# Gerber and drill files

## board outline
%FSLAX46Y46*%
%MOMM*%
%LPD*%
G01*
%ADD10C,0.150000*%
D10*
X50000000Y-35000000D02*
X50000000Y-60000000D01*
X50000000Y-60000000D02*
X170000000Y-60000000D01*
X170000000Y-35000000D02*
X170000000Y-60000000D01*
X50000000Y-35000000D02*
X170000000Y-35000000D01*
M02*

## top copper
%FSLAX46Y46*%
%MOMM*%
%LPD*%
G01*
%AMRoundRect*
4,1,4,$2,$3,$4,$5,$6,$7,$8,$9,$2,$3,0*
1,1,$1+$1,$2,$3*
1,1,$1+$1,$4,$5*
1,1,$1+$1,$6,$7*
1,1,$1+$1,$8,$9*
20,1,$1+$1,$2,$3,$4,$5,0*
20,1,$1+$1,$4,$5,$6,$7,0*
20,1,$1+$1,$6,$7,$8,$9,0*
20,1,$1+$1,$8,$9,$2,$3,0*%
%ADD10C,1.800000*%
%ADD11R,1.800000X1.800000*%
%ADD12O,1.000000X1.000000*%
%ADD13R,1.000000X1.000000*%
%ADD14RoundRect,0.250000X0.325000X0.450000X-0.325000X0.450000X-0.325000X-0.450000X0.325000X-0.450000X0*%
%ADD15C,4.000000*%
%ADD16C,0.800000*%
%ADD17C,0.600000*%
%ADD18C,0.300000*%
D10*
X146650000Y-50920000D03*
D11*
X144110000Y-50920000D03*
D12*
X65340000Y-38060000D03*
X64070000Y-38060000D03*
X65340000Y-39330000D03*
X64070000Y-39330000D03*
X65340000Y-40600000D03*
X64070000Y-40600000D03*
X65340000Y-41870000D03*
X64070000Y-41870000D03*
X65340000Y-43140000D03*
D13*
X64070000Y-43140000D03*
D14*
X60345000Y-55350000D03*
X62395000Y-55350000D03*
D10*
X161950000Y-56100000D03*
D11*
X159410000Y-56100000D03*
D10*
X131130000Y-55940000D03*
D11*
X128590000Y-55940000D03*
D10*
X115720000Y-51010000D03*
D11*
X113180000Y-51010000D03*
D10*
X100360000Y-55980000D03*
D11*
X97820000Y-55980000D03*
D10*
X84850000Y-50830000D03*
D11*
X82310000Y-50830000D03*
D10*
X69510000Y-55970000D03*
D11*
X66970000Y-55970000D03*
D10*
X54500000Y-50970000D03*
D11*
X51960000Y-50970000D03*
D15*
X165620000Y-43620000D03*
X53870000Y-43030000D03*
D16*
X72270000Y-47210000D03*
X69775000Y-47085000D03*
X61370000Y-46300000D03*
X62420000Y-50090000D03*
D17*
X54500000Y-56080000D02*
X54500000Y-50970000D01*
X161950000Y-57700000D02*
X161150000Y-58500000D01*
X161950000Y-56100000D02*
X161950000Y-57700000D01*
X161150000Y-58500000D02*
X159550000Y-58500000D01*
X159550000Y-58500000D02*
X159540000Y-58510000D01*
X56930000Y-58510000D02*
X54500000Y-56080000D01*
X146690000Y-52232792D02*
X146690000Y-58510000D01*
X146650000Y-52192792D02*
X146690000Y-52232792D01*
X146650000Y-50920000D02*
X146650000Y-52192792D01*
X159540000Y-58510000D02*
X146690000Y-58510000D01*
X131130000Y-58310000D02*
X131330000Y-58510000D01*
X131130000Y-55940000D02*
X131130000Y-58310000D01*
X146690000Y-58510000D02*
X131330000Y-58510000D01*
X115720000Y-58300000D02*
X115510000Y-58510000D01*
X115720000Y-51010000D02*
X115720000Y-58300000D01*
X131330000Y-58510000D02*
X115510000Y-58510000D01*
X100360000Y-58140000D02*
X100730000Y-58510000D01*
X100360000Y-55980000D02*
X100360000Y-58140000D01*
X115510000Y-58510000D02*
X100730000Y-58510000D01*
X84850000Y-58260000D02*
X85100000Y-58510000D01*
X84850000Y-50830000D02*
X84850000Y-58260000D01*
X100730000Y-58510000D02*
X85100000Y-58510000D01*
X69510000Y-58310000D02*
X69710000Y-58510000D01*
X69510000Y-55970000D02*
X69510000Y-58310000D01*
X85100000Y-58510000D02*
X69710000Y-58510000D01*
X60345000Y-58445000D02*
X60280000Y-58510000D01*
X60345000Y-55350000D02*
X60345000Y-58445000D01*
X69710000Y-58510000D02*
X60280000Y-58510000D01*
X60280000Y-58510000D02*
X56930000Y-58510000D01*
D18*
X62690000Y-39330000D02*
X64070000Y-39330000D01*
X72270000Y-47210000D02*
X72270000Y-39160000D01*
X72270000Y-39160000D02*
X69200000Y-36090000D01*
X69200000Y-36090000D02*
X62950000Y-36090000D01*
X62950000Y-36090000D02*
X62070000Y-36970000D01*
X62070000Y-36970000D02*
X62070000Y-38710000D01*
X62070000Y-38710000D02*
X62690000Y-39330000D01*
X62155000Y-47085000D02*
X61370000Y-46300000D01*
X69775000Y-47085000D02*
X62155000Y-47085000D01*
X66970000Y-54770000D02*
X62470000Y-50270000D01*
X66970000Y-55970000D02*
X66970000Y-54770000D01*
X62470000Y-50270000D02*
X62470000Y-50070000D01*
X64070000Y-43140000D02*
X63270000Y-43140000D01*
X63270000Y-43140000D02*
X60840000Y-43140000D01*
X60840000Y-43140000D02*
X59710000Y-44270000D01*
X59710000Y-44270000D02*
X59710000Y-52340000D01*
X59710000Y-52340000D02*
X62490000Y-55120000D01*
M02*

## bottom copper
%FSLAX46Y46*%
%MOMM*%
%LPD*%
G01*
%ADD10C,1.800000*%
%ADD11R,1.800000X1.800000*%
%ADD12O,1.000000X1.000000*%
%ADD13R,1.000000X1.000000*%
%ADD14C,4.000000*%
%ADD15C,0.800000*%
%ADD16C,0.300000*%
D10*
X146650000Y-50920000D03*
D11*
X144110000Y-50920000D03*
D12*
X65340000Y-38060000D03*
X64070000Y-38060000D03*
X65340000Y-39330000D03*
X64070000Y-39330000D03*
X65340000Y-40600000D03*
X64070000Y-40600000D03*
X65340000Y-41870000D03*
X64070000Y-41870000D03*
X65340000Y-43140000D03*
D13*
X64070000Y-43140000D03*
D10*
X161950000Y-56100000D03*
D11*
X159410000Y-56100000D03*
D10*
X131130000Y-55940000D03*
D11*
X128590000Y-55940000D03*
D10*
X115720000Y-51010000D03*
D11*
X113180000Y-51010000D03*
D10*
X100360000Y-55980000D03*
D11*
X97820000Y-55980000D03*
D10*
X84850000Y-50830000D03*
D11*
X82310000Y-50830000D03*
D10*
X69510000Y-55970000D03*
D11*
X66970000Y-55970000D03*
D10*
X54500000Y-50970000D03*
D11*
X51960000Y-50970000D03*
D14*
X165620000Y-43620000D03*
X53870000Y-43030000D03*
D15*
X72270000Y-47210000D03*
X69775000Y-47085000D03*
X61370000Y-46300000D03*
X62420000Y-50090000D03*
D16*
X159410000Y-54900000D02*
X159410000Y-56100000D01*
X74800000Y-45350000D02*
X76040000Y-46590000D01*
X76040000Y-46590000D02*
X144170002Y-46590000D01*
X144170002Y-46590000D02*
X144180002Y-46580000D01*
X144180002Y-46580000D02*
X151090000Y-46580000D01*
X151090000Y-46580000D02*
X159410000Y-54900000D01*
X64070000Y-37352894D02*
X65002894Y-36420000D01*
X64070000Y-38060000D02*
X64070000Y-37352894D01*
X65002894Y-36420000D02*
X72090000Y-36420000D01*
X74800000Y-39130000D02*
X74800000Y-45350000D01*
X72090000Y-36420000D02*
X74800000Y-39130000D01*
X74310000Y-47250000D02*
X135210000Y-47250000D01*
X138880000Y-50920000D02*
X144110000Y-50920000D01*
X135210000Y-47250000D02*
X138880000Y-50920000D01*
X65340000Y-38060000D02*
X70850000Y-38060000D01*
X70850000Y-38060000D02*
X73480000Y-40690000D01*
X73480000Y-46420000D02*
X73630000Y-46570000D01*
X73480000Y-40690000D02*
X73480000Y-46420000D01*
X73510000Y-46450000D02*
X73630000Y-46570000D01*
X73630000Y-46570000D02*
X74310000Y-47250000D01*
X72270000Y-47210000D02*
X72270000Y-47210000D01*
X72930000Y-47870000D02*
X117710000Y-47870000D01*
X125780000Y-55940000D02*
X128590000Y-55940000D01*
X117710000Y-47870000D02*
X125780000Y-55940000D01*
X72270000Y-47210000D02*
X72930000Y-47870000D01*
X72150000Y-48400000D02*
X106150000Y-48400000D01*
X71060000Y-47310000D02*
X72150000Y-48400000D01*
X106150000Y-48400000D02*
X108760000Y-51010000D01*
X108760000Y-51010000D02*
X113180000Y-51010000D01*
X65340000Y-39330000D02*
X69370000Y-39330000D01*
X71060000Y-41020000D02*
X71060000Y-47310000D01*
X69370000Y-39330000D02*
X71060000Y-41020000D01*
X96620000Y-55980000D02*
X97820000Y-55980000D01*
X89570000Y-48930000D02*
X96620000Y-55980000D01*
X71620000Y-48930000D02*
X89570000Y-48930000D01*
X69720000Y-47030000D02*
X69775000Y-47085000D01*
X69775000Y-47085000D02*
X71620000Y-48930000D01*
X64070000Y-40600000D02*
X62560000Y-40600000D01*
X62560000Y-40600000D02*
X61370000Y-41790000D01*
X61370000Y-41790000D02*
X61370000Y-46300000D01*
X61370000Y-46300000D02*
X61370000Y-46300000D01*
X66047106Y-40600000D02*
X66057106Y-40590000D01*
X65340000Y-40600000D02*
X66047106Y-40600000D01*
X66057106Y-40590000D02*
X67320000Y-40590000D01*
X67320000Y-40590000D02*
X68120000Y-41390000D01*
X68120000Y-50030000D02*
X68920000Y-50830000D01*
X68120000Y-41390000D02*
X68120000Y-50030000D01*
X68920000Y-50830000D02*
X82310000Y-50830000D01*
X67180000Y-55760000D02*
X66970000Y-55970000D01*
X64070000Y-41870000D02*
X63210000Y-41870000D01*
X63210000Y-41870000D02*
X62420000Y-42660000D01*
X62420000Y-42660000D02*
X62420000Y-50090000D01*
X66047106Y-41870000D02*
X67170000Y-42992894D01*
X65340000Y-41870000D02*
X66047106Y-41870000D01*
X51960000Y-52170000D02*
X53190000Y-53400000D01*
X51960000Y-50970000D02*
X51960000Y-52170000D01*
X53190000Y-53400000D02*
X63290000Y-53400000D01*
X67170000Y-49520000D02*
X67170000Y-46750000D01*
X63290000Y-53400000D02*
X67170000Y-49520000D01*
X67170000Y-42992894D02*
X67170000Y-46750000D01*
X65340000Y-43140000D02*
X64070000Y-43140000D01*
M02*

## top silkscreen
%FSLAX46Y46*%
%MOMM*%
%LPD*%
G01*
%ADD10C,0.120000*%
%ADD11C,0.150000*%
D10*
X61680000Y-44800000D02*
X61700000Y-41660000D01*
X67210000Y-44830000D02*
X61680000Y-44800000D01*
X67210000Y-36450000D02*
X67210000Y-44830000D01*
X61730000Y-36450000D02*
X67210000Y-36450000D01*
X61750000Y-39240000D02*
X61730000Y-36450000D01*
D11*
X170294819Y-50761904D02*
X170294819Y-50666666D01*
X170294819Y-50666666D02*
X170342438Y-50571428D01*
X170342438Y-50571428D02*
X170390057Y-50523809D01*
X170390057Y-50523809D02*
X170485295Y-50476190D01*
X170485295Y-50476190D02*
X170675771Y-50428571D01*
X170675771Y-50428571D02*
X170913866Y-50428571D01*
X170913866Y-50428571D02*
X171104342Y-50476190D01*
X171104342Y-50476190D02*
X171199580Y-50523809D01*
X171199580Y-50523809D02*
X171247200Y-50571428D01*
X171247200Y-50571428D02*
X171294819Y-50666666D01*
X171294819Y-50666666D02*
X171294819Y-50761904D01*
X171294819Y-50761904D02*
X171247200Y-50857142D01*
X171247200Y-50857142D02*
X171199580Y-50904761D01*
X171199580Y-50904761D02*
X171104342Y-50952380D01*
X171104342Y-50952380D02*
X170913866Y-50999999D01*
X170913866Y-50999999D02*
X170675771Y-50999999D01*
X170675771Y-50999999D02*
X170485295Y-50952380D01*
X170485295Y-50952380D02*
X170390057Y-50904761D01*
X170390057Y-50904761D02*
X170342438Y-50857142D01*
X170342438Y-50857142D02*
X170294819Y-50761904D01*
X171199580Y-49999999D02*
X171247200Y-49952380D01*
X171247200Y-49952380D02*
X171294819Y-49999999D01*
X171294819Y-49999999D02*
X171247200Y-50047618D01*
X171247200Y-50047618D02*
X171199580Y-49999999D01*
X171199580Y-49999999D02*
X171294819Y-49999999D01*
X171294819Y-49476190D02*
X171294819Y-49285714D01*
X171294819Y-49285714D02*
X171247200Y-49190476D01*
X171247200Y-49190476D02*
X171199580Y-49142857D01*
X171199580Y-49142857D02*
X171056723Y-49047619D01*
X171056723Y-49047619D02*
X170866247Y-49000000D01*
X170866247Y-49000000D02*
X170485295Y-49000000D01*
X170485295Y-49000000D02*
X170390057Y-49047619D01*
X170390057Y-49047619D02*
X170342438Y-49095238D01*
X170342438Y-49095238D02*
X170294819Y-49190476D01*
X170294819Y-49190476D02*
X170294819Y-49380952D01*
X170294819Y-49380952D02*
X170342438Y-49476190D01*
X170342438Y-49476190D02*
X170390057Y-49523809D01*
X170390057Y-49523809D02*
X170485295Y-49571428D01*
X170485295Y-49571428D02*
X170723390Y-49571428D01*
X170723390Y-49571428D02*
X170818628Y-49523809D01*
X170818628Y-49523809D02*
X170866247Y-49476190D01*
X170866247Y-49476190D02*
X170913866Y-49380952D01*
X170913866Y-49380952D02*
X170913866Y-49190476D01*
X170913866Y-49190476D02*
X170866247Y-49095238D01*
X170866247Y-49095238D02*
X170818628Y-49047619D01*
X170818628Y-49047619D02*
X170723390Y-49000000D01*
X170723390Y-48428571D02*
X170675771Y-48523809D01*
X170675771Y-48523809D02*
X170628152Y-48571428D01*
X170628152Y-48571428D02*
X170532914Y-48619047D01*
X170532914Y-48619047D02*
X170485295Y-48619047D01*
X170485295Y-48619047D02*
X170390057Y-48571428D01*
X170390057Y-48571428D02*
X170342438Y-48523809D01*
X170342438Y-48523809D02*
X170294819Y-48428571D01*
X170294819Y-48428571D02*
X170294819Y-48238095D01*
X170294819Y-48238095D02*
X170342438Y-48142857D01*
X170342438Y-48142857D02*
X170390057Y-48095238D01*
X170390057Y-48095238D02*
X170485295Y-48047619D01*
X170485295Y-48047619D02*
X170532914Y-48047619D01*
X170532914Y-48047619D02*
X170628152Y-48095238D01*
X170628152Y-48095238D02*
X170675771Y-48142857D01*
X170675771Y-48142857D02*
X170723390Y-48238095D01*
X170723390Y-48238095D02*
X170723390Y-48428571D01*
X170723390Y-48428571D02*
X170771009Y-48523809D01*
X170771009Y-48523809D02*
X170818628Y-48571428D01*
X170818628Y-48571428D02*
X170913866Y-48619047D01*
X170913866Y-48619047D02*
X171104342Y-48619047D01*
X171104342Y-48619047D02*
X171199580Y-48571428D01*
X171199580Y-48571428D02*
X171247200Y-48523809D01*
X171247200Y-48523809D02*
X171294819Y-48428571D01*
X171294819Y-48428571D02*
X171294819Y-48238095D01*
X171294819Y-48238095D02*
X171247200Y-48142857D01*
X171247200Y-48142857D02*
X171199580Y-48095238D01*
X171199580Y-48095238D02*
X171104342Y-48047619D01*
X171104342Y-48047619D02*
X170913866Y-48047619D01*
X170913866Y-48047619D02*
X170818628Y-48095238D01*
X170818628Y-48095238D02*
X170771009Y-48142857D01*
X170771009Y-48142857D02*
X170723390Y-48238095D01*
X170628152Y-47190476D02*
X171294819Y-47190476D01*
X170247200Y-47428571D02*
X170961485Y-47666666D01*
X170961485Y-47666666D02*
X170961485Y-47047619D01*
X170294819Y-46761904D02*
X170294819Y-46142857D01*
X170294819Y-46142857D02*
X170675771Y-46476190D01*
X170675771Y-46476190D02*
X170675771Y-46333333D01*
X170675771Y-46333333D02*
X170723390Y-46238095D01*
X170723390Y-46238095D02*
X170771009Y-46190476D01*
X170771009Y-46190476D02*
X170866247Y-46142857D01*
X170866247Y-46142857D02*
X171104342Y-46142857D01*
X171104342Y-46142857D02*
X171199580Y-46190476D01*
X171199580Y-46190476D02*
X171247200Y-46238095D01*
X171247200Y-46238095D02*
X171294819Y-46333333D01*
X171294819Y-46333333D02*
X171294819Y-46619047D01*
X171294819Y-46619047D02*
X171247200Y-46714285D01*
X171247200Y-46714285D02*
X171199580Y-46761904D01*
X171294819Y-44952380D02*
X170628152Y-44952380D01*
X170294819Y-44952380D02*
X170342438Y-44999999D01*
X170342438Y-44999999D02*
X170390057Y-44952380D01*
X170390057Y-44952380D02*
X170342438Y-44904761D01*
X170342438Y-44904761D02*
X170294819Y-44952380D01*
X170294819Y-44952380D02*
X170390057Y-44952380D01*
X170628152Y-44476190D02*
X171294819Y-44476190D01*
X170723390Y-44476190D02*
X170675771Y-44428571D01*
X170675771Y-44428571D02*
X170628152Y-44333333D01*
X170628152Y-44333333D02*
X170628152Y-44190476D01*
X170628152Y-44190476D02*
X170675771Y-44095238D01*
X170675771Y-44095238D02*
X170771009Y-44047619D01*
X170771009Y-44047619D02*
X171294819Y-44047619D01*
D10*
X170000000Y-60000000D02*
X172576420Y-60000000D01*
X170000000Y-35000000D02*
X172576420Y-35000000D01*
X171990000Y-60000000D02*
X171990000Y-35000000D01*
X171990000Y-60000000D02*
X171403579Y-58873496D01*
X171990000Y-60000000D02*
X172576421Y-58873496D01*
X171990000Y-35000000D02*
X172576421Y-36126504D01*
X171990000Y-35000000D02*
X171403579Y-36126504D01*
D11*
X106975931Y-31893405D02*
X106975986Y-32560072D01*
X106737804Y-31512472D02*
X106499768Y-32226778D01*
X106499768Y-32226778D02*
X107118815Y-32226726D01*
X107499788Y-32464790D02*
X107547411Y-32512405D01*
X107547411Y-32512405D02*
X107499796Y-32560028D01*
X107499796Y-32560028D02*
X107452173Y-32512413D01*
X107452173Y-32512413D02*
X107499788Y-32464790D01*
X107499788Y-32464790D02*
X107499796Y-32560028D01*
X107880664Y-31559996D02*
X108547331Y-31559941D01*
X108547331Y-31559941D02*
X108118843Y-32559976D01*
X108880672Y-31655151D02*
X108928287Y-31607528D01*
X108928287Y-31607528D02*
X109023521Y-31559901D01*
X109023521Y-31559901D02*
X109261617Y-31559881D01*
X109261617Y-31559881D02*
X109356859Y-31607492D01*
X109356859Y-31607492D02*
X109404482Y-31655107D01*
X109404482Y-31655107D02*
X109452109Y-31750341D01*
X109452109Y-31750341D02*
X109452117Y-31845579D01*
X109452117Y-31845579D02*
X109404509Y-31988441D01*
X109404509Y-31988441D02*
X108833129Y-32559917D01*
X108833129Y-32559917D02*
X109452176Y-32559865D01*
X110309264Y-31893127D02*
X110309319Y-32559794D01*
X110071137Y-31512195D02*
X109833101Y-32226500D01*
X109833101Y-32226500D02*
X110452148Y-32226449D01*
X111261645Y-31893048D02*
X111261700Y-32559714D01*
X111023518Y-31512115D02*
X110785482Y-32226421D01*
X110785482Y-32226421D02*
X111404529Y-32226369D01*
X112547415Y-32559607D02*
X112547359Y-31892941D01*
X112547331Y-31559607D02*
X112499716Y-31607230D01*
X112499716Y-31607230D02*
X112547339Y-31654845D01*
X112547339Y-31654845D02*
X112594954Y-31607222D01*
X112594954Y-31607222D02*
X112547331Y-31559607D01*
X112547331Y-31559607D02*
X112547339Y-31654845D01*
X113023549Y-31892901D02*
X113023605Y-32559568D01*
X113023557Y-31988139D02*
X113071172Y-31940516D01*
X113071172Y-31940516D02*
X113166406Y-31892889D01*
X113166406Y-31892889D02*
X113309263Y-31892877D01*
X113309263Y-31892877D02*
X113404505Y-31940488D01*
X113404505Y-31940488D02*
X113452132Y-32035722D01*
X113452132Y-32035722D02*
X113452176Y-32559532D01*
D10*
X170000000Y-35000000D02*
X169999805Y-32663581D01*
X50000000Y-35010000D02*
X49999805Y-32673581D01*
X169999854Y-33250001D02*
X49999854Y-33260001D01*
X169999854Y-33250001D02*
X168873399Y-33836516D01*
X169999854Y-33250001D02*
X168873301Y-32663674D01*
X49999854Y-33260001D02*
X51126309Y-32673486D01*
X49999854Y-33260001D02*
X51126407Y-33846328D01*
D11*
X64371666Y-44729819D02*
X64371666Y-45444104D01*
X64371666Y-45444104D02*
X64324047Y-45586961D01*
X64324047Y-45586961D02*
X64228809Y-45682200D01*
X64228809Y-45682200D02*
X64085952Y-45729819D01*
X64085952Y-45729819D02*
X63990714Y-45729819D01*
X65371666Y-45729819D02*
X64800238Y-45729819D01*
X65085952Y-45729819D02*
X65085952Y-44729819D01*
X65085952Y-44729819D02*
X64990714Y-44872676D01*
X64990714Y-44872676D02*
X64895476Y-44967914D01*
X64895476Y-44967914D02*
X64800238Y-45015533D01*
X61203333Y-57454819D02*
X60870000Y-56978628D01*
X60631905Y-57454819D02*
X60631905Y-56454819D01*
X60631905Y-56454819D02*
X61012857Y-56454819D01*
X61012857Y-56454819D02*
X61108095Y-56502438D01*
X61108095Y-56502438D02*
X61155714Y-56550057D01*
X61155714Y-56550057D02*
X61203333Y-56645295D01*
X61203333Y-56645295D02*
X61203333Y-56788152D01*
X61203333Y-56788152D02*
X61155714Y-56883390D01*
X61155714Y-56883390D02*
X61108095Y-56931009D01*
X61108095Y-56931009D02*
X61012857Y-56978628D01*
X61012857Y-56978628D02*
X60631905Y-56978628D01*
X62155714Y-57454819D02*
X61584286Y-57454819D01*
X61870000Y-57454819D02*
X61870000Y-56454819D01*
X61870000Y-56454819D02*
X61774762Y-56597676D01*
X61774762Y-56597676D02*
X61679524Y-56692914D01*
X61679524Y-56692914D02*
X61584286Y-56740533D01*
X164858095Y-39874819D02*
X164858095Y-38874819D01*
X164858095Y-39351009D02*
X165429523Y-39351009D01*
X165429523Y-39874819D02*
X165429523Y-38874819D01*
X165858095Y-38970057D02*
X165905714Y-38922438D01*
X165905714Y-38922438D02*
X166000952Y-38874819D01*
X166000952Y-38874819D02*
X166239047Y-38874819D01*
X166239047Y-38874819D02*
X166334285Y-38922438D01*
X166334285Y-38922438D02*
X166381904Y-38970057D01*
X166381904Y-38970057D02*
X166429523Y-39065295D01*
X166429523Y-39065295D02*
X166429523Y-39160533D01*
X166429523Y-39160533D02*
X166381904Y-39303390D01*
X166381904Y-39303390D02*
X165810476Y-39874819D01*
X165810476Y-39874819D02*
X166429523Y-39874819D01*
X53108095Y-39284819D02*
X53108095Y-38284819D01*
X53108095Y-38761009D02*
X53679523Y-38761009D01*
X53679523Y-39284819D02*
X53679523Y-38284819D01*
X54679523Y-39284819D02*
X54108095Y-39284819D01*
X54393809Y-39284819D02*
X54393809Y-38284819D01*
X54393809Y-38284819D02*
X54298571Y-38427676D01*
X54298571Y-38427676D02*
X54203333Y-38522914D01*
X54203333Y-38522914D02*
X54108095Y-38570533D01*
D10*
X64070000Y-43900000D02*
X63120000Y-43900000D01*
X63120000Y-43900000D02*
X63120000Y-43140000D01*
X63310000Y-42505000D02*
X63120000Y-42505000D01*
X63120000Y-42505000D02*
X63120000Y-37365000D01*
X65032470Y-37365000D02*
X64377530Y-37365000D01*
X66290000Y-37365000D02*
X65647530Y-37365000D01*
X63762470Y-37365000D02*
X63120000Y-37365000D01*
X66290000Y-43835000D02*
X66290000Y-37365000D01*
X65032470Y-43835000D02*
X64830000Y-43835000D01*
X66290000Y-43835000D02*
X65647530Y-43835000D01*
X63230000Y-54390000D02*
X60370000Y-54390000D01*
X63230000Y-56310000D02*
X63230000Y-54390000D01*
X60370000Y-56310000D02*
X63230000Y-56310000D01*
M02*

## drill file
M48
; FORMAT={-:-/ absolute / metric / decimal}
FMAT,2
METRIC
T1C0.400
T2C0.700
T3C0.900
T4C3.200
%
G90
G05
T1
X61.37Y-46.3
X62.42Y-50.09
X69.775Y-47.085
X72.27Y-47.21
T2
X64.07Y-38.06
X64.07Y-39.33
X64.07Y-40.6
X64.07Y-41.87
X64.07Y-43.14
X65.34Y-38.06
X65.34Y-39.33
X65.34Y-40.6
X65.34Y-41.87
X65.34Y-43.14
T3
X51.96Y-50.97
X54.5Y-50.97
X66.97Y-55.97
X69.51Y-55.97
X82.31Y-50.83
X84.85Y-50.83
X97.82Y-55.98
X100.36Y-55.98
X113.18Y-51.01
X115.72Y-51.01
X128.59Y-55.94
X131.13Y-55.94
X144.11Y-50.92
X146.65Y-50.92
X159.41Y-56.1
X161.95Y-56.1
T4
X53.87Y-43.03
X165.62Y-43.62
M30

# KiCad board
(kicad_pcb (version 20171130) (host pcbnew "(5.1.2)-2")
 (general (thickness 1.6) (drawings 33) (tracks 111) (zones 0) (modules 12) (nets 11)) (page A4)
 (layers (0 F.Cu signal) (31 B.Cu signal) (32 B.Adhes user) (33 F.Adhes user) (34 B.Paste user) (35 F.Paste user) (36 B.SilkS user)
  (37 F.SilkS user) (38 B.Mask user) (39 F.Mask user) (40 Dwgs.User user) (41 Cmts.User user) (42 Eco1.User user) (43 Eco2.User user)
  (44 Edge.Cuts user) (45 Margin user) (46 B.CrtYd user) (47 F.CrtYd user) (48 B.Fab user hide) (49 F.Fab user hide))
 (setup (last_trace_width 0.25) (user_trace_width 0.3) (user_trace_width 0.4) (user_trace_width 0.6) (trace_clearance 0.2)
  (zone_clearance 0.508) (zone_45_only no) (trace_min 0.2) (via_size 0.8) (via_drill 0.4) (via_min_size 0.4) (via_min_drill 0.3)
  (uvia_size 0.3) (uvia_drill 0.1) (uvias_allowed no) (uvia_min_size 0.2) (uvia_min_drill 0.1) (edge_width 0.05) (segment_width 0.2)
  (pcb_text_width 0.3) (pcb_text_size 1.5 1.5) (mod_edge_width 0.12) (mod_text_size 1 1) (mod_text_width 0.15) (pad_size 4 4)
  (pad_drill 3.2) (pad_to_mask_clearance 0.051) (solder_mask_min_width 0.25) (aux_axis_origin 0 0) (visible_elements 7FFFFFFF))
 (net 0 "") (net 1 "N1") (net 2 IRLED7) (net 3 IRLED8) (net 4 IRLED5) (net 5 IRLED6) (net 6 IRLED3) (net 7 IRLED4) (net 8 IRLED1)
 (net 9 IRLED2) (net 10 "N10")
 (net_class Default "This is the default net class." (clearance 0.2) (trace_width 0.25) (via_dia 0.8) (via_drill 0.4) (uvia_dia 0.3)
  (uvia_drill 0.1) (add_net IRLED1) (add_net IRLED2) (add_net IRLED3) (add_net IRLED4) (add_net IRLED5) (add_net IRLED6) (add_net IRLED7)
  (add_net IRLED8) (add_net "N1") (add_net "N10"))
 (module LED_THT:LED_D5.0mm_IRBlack (layer B.Cu) (at 144.11 50.92)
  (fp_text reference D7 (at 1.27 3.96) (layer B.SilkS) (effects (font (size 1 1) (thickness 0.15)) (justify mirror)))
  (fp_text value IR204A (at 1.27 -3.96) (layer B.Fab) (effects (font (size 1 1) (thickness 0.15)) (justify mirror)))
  (pad 2 thru_hole circle (at 2.54 0) (size 1.8 1.8) (drill 0.9) (layers *.Cu *.Mask) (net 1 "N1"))
  (pad 1 thru_hole rect (at 0 0) (size 1.8 1.8) (drill 0.9) (layers *.Cu *.Mask) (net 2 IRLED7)))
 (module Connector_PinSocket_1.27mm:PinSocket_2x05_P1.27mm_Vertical (layer F.Cu) (at 64.07 43.14 180)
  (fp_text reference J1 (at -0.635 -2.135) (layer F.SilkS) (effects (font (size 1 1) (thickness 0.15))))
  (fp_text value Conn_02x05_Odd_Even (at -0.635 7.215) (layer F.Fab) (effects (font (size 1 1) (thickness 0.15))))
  (fp_line (start 0 -0.76) (end 0.95 -0.76) (layer F.SilkS) (width 0.12))
  (fp_line (start 0.95 -0.76) (end 0.95 0) (layer F.SilkS) (width 0.12))
  (fp_line (start 0.76 0.635) (end 0.95 0.635) (layer F.SilkS) (width 0.12))
  (fp_line (start 0.95 0.635) (end 0.95 5.775) (layer F.SilkS) (width 0.12))
  (fp_line (start -0.96247 5.775) (end -0.30753 5.775) (layer F.SilkS) (width 0.12))
  (fp_line (start -2.22 5.775) (end -1.57753 5.775) (layer F.SilkS) (width 0.12))
  (fp_line (start 0.30753 5.775) (end 0.95 5.775) (layer F.SilkS) (width 0.12))
  (fp_line (start -2.22 -0.695) (end -2.22 5.775) (layer F.SilkS) (width 0.12))
  (fp_line (start -0.96247 -0.695) (end -0.76 -0.695) (layer F.SilkS) (width 0.12))
  (fp_line (start -2.22 -0.695) (end -1.57753 -0.695) (layer F.SilkS) (width 0.12))
  (pad 10 thru_hole oval (at -1.27 5.08 180) (size 1 1) (drill 0.7) (layers *.Cu *.Mask) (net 2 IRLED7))
  (pad 9 thru_hole oval (at 0 5.08 180) (size 1 1) (drill 0.7) (layers *.Cu *.Mask) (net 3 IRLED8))
  (pad 8 thru_hole oval (at -1.27 3.81 180) (size 1 1) (drill 0.7) (layers *.Cu *.Mask) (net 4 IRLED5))
  (pad 7 thru_hole oval (at 0 3.81 180) (size 1 1) (drill 0.7) (layers *.Cu *.Mask) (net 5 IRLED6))
  (pad 6 thru_hole oval (at -1.27 2.54 180) (size 1 1) (drill 0.7) (layers *.Cu *.Mask) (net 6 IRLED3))
  (pad 5 thru_hole oval (at 0 2.54 180) (size 1 1) (drill 0.7) (layers *.Cu *.Mask) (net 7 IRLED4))
  (pad 4 thru_hole oval (at -1.27 1.27 180) (size 1 1) (drill 0.7) (layers *.Cu *.Mask) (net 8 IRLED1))
  (pad 3 thru_hole oval (at 0 1.27 180) (size 1 1) (drill 0.7) (layers *.Cu *.Mask) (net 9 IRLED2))
  (pad 2 thru_hole oval (at -1.27 0 180) (size 1 1) (drill 0.7) (layers *.Cu *.Mask) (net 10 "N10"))
  (pad 1 thru_hole rect (at 0 0 180) (size 1 1) (drill 0.7) (layers *.Cu *.Mask) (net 10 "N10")))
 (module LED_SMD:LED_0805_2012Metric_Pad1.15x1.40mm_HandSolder (layer F.Cu) (at 61.37 55.35 180)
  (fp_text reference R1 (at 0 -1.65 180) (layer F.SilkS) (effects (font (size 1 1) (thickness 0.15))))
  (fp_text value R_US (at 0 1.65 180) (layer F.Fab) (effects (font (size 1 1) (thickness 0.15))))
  (fp_line (start -1.86 0.96) (end 1 0.96) (layer F.SilkS) (width 0.12))
  (fp_line (start -1.86 -0.96) (end -1.86 0.96) (layer F.SilkS) (width 0.12))
  (fp_line (start 1 -0.96) (end -1.86 -0.96) (layer F.SilkS) (width 0.12))
  (pad 2 smd roundrect (at 1.025 0 180) (size 1.15 1.4) (layers F.Cu F.Paste F.Mask) (roundrect_rratio 0.217391) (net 1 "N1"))
  (pad 1 smd roundrect (at -1.025 0 180) (size 1.15 1.4) (layers F.Cu F.Paste F.Mask) (roundrect_rratio 0.217391) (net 10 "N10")))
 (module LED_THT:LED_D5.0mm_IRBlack (layer B.Cu) (at 159.41 56.1)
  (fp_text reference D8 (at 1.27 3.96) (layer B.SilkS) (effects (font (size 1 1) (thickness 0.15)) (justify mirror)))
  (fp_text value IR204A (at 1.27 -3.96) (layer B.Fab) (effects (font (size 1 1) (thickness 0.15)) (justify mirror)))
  (pad 2 thru_hole circle (at 2.54 0) (size 1.8 1.8) (drill 0.9) (layers *.Cu *.Mask) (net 1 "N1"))
  (pad 1 thru_hole rect (at 0 0) (size 1.8 1.8) (drill 0.9) (layers *.Cu *.Mask) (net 3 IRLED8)))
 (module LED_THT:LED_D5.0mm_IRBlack (layer B.Cu) (at 128.59 55.94)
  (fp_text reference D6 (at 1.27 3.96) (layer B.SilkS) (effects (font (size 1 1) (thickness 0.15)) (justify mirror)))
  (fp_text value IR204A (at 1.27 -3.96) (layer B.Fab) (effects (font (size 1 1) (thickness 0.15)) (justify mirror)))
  (pad 2 thru_hole circle (at 2.54 0) (size 1.8 1.8) (drill 0.9) (layers *.Cu *.Mask) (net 1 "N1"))
  (pad 1 thru_hole rect (at 0 0) (size 1.8 1.8) (drill 0.9) (layers *.Cu *.Mask) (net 5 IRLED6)))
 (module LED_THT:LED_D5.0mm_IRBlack (layer B.Cu) (at 113.18 51.01)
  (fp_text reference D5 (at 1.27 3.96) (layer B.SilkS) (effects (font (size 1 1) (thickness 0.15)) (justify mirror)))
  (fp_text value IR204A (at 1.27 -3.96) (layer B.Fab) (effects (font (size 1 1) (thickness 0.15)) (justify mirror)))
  (pad 2 thru_hole circle (at 2.54 0) (size 1.8 1.8) (drill 0.9) (layers *.Cu *.Mask) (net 1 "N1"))
  (pad 1 thru_hole rect (at 0 0) (size 1.8 1.8) (drill 0.9) (layers *.Cu *.Mask) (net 4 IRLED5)))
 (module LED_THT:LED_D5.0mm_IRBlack (layer B.Cu) (at 97.82 55.98)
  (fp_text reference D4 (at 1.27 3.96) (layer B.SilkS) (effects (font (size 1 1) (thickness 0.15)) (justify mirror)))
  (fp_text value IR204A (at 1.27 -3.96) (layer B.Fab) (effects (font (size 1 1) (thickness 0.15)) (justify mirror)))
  (pad 2 thru_hole circle (at 2.54 0) (size 1.8 1.8) (drill 0.9) (layers *.Cu *.Mask) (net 1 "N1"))
  (pad 1 thru_hole rect (at 0 0) (size 1.8 1.8) (drill 0.9) (layers *.Cu *.Mask) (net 7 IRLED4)))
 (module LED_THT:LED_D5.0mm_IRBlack (layer B.Cu) (at 82.31 50.83)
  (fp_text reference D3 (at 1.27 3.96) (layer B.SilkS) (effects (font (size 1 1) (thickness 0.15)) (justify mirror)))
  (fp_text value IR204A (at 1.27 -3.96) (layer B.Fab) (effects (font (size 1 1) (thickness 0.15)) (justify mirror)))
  (pad 2 thru_hole circle (at 2.54 0) (size 1.8 1.8) (drill 0.9) (layers *.Cu *.Mask) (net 1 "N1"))
  (pad 1 thru_hole rect (at 0 0) (size 1.8 1.8) (drill 0.9) (layers *.Cu *.Mask) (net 6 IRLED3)))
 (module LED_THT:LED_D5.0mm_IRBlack (layer B.Cu) (at 66.97 55.97)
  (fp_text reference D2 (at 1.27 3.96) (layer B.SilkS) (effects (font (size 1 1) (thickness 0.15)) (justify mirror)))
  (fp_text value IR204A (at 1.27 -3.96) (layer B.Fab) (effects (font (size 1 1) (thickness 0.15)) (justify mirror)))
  (pad 2 thru_hole circle (at 2.54 0) (size 1.8 1.8) (drill 0.9) (layers *.Cu *.Mask) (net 1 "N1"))
  (pad 1 thru_hole rect (at 0 0) (size 1.8 1.8) (drill 0.9) (layers *.Cu *.Mask) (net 9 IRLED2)))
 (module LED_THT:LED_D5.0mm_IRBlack (layer B.Cu) (at 51.96 50.97)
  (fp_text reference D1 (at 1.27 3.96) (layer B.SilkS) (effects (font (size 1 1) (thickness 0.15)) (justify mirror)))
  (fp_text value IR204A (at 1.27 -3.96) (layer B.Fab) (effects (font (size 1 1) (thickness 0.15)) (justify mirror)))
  (pad 2 thru_hole circle (at 2.54 0) (size 1.8 1.8) (drill 0.9) (layers *.Cu *.Mask) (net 1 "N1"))
  (pad 1 thru_hole rect (at 0 0) (size 1.8 1.8) (drill 0.9) (layers *.Cu *.Mask) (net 8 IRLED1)))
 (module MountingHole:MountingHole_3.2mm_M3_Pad (layer F.Cu) (at 165.62 43.62)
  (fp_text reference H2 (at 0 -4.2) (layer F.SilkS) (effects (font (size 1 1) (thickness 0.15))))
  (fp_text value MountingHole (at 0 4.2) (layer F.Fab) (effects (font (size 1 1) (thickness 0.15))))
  (pad 1 thru_hole circle (at 0 0) (size 4 4) (drill 3.2) (layers *.Cu *.Mask)))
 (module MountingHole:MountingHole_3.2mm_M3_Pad (layer F.Cu) (at 53.87 43.03)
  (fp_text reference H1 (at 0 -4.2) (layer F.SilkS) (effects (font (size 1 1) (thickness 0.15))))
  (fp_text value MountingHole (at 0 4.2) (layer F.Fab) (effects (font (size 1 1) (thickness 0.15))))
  (pad 1 thru_hole circle (at 0 0) (size 4 4) (drill 3.2) (layers *.Cu *.Mask)))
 (gr_line (start 61.68 44.8) (end 61.7 41.66) (layer F.SilkS) (width 0.12))
 (gr_line (start 67.21 44.83) (end 61.68 44.8) (layer F.SilkS) (width 0.12))
 (gr_line (start 67.21 36.45) (end 67.21 44.83) (layer F.SilkS) (width 0.12))
 (gr_line (start 61.73 36.45) (end 67.21 36.45) (layer F.SilkS) (width 0.12))
 (gr_line (start 61.75 39.24) (end 61.73 36.45) (layer F.SilkS) (width 0.12))
 (gr_line (start 50 35) (end 50 60) (layer Edge.Cuts) (width 0.15))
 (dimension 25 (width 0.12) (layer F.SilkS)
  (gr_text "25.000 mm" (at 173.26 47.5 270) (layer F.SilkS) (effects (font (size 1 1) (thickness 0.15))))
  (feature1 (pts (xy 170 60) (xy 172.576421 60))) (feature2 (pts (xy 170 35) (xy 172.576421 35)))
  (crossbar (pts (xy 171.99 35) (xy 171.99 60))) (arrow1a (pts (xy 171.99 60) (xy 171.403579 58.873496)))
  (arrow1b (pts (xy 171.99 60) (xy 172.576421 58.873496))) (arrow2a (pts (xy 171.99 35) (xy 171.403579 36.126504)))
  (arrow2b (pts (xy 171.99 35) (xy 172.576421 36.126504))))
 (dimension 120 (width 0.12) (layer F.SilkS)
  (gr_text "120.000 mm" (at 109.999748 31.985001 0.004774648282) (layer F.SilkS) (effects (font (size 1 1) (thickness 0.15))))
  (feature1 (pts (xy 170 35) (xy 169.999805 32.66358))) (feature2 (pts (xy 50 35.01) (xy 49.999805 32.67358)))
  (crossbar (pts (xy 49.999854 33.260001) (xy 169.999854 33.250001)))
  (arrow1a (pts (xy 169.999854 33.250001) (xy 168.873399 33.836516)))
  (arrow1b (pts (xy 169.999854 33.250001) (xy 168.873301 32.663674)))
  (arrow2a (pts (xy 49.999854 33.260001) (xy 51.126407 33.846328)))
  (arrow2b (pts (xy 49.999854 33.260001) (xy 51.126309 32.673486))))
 (gr_line (start 50 60) (end 170 60) (layer Edge.Cuts) (width 0.15))
 (gr_line (start 170 35) (end 170 60) (layer Edge.Cuts) (width 0.15))
 (gr_line (start 50 35) (end 170 35) (layer Edge.Cuts) (width 0.15))
 (segment (start 54.5 56.08) (end 54.5 50.97) (width 0.6) (layer F.Cu) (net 1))
 (segment (start 161.95 57.7) (end 161.15 58.5) (width 0.6) (layer F.Cu) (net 1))
 (segment (start 161.95 56.1) (end 161.95 57.7) (width 0.6) (layer F.Cu) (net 1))
 (segment (start 161.15 58.5) (end 159.55 58.5) (width 0.6) (layer F.Cu) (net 1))
 (segment (start 159.55 58.5) (end 159.54 58.51) (width 0.6) (layer F.Cu) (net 1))
 (segment (start 56.93 58.51) (end 54.5 56.08) (width 0.6) (layer F.Cu) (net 1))
 (segment (start 146.69 52.232792) (end 146.69 58.51) (width 0.6) (layer F.Cu) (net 1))
 (segment (start 146.65 52.192792) (end 146.69 52.232792) (width 0.6) (layer F.Cu) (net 1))
 (segment (start 146.65 50.92) (end 146.65 52.192792) (width 0.6) (layer F.Cu) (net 1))
 (segment (start 159.54 58.51) (end 146.69 58.51) (width 0.6) (layer F.Cu) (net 1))
 (segment (start 131.13 58.31) (end 131.33 58.51) (width 0.6) (layer F.Cu) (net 1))
 (segment (start 131.13 55.94) (end 131.13 58.31) (width 0.6) (layer F.Cu) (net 1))
 (segment (start 146.69 58.51) (end 131.33 58.51) (width 0.6) (layer F.Cu) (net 1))
 (segment (start 115.72 58.3) (end 115.51 58.51) (width 0.6) (layer F.Cu) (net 1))
 (segment (start 115.72 51.01) (end 115.72 58.3) (width 0.6) (layer F.Cu) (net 1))
 (segment (start 131.33 58.51) (end 115.51 58.51) (width 0.6) (layer F.Cu) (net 1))
 (segment (start 100.36 58.14) (end 100.73 58.51) (width 0.6) (layer F.Cu) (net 1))
 (segment (start 100.36 55.98) (end 100.36 58.14) (width 0.6) (layer F.Cu) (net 1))
 (segment (start 115.51 58.51) (end 100.73 58.51) (width 0.6) (layer F.Cu) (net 1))
 (segment (start 84.85 58.26) (end 85.1 58.51) (width 0.6) (layer F.Cu) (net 1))
 (segment (start 84.85 50.83) (end 84.85 58.26) (width 0.6) (layer F.Cu) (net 1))
 (segment (start 100.73 58.51) (end 85.1 58.51) (width 0.6) (layer F.Cu) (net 1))
 (segment (start 69.51 58.31) (end 69.71 58.51) (width 0.6) (layer F.Cu) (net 1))
 (segment (start 69.51 55.97) (end 69.51 58.31) (width 0.6) (layer F.Cu) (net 1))
 (segment (start 85.1 58.51) (end 69.71 58.51) (width 0.6) (layer F.Cu) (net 1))
 (segment (start 60.345 58.445) (end 60.28 58.51) (width 0.6) (layer F.Cu) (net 1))
 (segment (start 60.345 55.35) (end 60.345 58.445) (width 0.6) (layer F.Cu) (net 1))
 (segment (start 69.71 58.51) (end 60.28 58.51) (width 0.6) (layer F.Cu) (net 1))
 (segment (start 60.28 58.51) (end 56.93 58.51) (width 0.6) (layer F.Cu) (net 1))
 (segment (start 159.41 54.9) (end 159.41 56.1) (width 0.3) (layer B.Cu) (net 3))
 (segment (start 74.8 45.35) (end 76.04 46.59) (width 0.3) (layer B.Cu) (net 3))
 (segment (start 76.04 46.59) (end 144.170002 46.59) (width 0.3) (layer B.Cu) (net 3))
 (segment (start 144.170002 46.59) (end 144.180002 46.58) (width 0.3) (layer B.Cu) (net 3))
 (segment (start 144.180002 46.58) (end 151.09 46.58) (width 0.3) (layer B.Cu) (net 3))
 (segment (start 151.09 46.58) (end 159.41 54.9) (width 0.3) (layer B.Cu) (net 3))
 (segment (start 64.07 37.352894) (end 65.002894 36.42) (width 0.3) (layer B.Cu) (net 3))
 (segment (start 64.07 38.06) (end 64.07 37.352894) (width 0.3) (layer B.Cu) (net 3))
 (segment (start 65.002894 36.42) (end 72.09 36.42) (width 0.3) (layer B.Cu) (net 3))
 (segment (start 74.8 39.13) (end 74.8 45.35) (width 0.3) (layer B.Cu) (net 3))
 (segment (start 72.09 36.42) (end 74.8 39.13) (width 0.3) (layer B.Cu) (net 3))
 (segment (start 74.31 47.25) (end 135.21 47.25) (width 0.3) (layer B.Cu) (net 2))
 (segment (start 138.88 50.92) (end 144.11 50.92) (width 0.3) (layer B.Cu) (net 2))
 (segment (start 135.21 47.25) (end 138.88 50.92) (width 0.3) (layer B.Cu) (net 2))
 (segment (start 65.34 38.06) (end 70.85 38.06) (width 0.3) (layer B.Cu) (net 2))
 (segment (start 70.85 38.06) (end 73.48 40.69) (width 0.3) (layer B.Cu) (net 2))
 (segment (start 73.48 46.42) (end 73.63 46.57) (width 0.3) (layer B.Cu) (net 2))
 (segment (start 73.48 40.69) (end 73.48 46.42) (width 0.3) (layer B.Cu) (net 2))
 (segment (start 73.51 46.45) (end 73.63 46.57) (width 0.3) (layer B.Cu) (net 2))
 (segment (start 73.63 46.57) (end 74.31 47.25) (width 0.3) (layer B.Cu) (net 2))
 (segment (start 72.27 47.21) (end 72.27 47.21) (width 0.3) (layer B.Cu) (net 5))
 (segment (start 72.93 47.87) (end 117.71 47.87) (width 0.3) (layer B.Cu) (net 5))
 (segment (start 125.78 55.94) (end 128.59 55.94) (width 0.3) (layer B.Cu) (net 5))
 (segment (start 117.71 47.87) (end 125.78 55.94) (width 0.3) (layer B.Cu) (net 5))
 (segment (start 72.27 47.21) (end 72.93 47.87) (width 0.3) (layer B.Cu) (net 5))
 (via (at 72.27 47.21) (size 0.8) (drill 0.4) (layers F.Cu B.Cu) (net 5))
 (segment (start 62.69 39.33) (end 64.07 39.33) (width 0.3) (layer F.Cu) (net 5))
 (segment (start 72.27 47.21) (end 72.27 39.16) (width 0.3) (layer F.Cu) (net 5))
 (segment (start 72.27 39.16) (end 69.2 36.09) (width 0.3) (layer F.Cu) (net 5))
 (segment (start 69.2 36.09) (end 62.95 36.09) (width 0.3) (layer F.Cu) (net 5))
 (segment (start 62.95 36.09) (end 62.07 36.97) (width 0.3) (layer F.Cu) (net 5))
 (segment (start 62.07 36.97) (end 62.07 38.71) (width 0.3) (layer F.Cu) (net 5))
 (segment (start 62.07 38.71) (end 62.69 39.33) (width 0.3) (layer F.Cu) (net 5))
 (segment (start 72.15 48.4) (end 106.15 48.4) (width 0.3) (layer B.Cu) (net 4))
 (segment (start 71.06 47.31) (end 72.15 48.4) (width 0.3) (layer B.Cu) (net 4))
 (segment (start 106.15 48.4) (end 108.76 51.01) (width 0.3) (layer B.Cu) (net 4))
 (segment (start 108.76 51.01) (end 113.18 51.01) (width 0.3) (layer B.Cu) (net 4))
 (segment (start 65.34 39.33) (end 69.37 39.33) (width 0.3) (layer B.Cu) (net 4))
 (segment (start 71.06 41.02) (end 71.06 47.31) (width 0.3) (layer B.Cu) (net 4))
 (segment (start 69.37 39.33) (end 71.06 41.02) (width 0.3) (layer B.Cu) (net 4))
 (segment (start 96.62 55.98) (end 97.82 55.98) (width 0.3) (layer B.Cu) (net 7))
 (segment (start 89.57 48.93) (end 96.62 55.98) (width 0.3) (layer B.Cu) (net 7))
 (segment (start 71.62 48.93) (end 89.57 48.93) (width 0.3) (layer B.Cu) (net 7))
 (segment (start 69.72 47.03) (end 69.775 47.085) (width 0.3) (layer B.Cu) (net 7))
 (segment (start 69.775 47.085) (end 71.62 48.93) (width 0.3) (layer B.Cu) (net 7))
 (via (at 69.775 47.085) (size 0.8) (drill 0.4) (layers F.Cu B.Cu) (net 7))
 (segment (start 64.07 40.6) (end 62.56 40.6) (width 0.3) (layer B.Cu) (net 7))
 (segment (start 62.56 40.6) (end 61.37 41.79) (width 0.3) (layer B.Cu) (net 7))
 (segment (start 61.37 41.79) (end 61.37 46.3) (width 0.3) (layer B.Cu) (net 7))
 (segment (start 61.37 46.3) (end 61.37 46.3) (width 0.3) (layer B.Cu) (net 7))
 (via (at 61.37 46.3) (size 0.8) (drill 0.4) (layers F.Cu B.Cu) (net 7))
 (segment (start 62.155 47.085) (end 61.37 46.3) (width 0.3) (layer F.Cu) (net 7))
 (segment (start 69.775 47.085) (end 62.155 47.085) (width 0.3) (layer F.Cu) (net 7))
 (segment (start 66.047106 40.6) (end 66.057106 40.59) (width 0.3) (layer B.Cu) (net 6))
 (segment (start 65.34 40.6) (end 66.047106 40.6) (width 0.3) (layer B.Cu) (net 6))
 (segment (start 66.057106 40.59) (end 67.32 40.59) (width 0.3) (layer B.Cu) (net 6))
 (segment (start 67.32 40.59) (end 68.12 41.39) (width 0.3) (layer B.Cu) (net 6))
 (segment (start 68.12 50.03) (end 68.92 50.83) (width 0.3) (layer B.Cu) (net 6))
 (segment (start 68.12 41.39) (end 68.12 50.03) (width 0.3) (layer B.Cu) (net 6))
 (segment (start 68.92 50.83) (end 82.31 50.83) (width 0.3) (layer B.Cu) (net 6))
 (segment (start 67.18 55.76) (end 66.97 55.97) (width 0.3) (layer B.Cu) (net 9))
 (segment (start 64.07 41.87) (end 63.21 41.87) (width 0.3) (layer B.Cu) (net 9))
 (segment (start 63.21 41.87) (end 62.42 42.66) (width 0.3) (layer B.Cu) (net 9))
 (segment (start 62.42 42.66) (end 62.42 50.09) (width 0.3) (layer B.Cu) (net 9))
 (segment (start 66.97 54.77) (end 62.47 50.27) (width 0.3) (layer F.Cu) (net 9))
 (segment (start 66.97 55.97) (end 66.97 54.77) (width 0.3) (layer F.Cu) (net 9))
 (segment (start 62.47 50.27) (end 62.47 50.07) (width 0.3) (layer F.Cu) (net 9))
 (via (at 62.42 50.09) (size 0.8) (drill 0.4) (layers F.Cu B.Cu) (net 9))
 (segment (start 66.047106 41.87) (end 67.17 42.992894) (width 0.3) (layer B.Cu) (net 8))
 (segment (start 65.34 41.87) (end 66.047106 41.87) (width 0.3) (layer B.Cu) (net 8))
 (segment (start 51.96 52.17) (end 53.19 53.4) (width 0.3) (layer B.Cu) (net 8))
 (segment (start 51.96 50.97) (end 51.96 52.17) (width 0.3) (layer B.Cu) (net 8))
 (segment (start 53.19 53.4) (end 63.29 53.4) (width 0.3) (layer B.Cu) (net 8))
 (segment (start 67.17 49.52) (end 67.17 46.75) (width 0.3) (layer B.Cu) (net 8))
 (segment (start 63.29 53.4) (end 67.17 49.52) (width 0.3) (layer B.Cu) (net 8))
 (segment (start 67.17 42.992894) (end 67.17 46.75) (width 0.3) (layer B.Cu) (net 8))
 (segment (start 65.34 43.14) (end 64.07 43.14) (width 0.3) (layer B.Cu) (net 10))
 (segment (start 64.07 43.14) (end 63.27 43.14) (width 0.3) (layer F.Cu) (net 10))
 (segment (start 63.27 43.14) (end 60.84 43.14) (width 0.3) (layer F.Cu) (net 10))
 (segment (start 60.84 43.14) (end 59.71 44.27) (width 0.3) (layer F.Cu) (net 10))
 (segment (start 59.71 44.27) (end 59.71 52.34) (width 0.3) (layer F.Cu) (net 10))
 (segment (start 59.71 52.34) (end 62.49 55.12) (width 0.3) (layer F.Cu) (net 10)))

